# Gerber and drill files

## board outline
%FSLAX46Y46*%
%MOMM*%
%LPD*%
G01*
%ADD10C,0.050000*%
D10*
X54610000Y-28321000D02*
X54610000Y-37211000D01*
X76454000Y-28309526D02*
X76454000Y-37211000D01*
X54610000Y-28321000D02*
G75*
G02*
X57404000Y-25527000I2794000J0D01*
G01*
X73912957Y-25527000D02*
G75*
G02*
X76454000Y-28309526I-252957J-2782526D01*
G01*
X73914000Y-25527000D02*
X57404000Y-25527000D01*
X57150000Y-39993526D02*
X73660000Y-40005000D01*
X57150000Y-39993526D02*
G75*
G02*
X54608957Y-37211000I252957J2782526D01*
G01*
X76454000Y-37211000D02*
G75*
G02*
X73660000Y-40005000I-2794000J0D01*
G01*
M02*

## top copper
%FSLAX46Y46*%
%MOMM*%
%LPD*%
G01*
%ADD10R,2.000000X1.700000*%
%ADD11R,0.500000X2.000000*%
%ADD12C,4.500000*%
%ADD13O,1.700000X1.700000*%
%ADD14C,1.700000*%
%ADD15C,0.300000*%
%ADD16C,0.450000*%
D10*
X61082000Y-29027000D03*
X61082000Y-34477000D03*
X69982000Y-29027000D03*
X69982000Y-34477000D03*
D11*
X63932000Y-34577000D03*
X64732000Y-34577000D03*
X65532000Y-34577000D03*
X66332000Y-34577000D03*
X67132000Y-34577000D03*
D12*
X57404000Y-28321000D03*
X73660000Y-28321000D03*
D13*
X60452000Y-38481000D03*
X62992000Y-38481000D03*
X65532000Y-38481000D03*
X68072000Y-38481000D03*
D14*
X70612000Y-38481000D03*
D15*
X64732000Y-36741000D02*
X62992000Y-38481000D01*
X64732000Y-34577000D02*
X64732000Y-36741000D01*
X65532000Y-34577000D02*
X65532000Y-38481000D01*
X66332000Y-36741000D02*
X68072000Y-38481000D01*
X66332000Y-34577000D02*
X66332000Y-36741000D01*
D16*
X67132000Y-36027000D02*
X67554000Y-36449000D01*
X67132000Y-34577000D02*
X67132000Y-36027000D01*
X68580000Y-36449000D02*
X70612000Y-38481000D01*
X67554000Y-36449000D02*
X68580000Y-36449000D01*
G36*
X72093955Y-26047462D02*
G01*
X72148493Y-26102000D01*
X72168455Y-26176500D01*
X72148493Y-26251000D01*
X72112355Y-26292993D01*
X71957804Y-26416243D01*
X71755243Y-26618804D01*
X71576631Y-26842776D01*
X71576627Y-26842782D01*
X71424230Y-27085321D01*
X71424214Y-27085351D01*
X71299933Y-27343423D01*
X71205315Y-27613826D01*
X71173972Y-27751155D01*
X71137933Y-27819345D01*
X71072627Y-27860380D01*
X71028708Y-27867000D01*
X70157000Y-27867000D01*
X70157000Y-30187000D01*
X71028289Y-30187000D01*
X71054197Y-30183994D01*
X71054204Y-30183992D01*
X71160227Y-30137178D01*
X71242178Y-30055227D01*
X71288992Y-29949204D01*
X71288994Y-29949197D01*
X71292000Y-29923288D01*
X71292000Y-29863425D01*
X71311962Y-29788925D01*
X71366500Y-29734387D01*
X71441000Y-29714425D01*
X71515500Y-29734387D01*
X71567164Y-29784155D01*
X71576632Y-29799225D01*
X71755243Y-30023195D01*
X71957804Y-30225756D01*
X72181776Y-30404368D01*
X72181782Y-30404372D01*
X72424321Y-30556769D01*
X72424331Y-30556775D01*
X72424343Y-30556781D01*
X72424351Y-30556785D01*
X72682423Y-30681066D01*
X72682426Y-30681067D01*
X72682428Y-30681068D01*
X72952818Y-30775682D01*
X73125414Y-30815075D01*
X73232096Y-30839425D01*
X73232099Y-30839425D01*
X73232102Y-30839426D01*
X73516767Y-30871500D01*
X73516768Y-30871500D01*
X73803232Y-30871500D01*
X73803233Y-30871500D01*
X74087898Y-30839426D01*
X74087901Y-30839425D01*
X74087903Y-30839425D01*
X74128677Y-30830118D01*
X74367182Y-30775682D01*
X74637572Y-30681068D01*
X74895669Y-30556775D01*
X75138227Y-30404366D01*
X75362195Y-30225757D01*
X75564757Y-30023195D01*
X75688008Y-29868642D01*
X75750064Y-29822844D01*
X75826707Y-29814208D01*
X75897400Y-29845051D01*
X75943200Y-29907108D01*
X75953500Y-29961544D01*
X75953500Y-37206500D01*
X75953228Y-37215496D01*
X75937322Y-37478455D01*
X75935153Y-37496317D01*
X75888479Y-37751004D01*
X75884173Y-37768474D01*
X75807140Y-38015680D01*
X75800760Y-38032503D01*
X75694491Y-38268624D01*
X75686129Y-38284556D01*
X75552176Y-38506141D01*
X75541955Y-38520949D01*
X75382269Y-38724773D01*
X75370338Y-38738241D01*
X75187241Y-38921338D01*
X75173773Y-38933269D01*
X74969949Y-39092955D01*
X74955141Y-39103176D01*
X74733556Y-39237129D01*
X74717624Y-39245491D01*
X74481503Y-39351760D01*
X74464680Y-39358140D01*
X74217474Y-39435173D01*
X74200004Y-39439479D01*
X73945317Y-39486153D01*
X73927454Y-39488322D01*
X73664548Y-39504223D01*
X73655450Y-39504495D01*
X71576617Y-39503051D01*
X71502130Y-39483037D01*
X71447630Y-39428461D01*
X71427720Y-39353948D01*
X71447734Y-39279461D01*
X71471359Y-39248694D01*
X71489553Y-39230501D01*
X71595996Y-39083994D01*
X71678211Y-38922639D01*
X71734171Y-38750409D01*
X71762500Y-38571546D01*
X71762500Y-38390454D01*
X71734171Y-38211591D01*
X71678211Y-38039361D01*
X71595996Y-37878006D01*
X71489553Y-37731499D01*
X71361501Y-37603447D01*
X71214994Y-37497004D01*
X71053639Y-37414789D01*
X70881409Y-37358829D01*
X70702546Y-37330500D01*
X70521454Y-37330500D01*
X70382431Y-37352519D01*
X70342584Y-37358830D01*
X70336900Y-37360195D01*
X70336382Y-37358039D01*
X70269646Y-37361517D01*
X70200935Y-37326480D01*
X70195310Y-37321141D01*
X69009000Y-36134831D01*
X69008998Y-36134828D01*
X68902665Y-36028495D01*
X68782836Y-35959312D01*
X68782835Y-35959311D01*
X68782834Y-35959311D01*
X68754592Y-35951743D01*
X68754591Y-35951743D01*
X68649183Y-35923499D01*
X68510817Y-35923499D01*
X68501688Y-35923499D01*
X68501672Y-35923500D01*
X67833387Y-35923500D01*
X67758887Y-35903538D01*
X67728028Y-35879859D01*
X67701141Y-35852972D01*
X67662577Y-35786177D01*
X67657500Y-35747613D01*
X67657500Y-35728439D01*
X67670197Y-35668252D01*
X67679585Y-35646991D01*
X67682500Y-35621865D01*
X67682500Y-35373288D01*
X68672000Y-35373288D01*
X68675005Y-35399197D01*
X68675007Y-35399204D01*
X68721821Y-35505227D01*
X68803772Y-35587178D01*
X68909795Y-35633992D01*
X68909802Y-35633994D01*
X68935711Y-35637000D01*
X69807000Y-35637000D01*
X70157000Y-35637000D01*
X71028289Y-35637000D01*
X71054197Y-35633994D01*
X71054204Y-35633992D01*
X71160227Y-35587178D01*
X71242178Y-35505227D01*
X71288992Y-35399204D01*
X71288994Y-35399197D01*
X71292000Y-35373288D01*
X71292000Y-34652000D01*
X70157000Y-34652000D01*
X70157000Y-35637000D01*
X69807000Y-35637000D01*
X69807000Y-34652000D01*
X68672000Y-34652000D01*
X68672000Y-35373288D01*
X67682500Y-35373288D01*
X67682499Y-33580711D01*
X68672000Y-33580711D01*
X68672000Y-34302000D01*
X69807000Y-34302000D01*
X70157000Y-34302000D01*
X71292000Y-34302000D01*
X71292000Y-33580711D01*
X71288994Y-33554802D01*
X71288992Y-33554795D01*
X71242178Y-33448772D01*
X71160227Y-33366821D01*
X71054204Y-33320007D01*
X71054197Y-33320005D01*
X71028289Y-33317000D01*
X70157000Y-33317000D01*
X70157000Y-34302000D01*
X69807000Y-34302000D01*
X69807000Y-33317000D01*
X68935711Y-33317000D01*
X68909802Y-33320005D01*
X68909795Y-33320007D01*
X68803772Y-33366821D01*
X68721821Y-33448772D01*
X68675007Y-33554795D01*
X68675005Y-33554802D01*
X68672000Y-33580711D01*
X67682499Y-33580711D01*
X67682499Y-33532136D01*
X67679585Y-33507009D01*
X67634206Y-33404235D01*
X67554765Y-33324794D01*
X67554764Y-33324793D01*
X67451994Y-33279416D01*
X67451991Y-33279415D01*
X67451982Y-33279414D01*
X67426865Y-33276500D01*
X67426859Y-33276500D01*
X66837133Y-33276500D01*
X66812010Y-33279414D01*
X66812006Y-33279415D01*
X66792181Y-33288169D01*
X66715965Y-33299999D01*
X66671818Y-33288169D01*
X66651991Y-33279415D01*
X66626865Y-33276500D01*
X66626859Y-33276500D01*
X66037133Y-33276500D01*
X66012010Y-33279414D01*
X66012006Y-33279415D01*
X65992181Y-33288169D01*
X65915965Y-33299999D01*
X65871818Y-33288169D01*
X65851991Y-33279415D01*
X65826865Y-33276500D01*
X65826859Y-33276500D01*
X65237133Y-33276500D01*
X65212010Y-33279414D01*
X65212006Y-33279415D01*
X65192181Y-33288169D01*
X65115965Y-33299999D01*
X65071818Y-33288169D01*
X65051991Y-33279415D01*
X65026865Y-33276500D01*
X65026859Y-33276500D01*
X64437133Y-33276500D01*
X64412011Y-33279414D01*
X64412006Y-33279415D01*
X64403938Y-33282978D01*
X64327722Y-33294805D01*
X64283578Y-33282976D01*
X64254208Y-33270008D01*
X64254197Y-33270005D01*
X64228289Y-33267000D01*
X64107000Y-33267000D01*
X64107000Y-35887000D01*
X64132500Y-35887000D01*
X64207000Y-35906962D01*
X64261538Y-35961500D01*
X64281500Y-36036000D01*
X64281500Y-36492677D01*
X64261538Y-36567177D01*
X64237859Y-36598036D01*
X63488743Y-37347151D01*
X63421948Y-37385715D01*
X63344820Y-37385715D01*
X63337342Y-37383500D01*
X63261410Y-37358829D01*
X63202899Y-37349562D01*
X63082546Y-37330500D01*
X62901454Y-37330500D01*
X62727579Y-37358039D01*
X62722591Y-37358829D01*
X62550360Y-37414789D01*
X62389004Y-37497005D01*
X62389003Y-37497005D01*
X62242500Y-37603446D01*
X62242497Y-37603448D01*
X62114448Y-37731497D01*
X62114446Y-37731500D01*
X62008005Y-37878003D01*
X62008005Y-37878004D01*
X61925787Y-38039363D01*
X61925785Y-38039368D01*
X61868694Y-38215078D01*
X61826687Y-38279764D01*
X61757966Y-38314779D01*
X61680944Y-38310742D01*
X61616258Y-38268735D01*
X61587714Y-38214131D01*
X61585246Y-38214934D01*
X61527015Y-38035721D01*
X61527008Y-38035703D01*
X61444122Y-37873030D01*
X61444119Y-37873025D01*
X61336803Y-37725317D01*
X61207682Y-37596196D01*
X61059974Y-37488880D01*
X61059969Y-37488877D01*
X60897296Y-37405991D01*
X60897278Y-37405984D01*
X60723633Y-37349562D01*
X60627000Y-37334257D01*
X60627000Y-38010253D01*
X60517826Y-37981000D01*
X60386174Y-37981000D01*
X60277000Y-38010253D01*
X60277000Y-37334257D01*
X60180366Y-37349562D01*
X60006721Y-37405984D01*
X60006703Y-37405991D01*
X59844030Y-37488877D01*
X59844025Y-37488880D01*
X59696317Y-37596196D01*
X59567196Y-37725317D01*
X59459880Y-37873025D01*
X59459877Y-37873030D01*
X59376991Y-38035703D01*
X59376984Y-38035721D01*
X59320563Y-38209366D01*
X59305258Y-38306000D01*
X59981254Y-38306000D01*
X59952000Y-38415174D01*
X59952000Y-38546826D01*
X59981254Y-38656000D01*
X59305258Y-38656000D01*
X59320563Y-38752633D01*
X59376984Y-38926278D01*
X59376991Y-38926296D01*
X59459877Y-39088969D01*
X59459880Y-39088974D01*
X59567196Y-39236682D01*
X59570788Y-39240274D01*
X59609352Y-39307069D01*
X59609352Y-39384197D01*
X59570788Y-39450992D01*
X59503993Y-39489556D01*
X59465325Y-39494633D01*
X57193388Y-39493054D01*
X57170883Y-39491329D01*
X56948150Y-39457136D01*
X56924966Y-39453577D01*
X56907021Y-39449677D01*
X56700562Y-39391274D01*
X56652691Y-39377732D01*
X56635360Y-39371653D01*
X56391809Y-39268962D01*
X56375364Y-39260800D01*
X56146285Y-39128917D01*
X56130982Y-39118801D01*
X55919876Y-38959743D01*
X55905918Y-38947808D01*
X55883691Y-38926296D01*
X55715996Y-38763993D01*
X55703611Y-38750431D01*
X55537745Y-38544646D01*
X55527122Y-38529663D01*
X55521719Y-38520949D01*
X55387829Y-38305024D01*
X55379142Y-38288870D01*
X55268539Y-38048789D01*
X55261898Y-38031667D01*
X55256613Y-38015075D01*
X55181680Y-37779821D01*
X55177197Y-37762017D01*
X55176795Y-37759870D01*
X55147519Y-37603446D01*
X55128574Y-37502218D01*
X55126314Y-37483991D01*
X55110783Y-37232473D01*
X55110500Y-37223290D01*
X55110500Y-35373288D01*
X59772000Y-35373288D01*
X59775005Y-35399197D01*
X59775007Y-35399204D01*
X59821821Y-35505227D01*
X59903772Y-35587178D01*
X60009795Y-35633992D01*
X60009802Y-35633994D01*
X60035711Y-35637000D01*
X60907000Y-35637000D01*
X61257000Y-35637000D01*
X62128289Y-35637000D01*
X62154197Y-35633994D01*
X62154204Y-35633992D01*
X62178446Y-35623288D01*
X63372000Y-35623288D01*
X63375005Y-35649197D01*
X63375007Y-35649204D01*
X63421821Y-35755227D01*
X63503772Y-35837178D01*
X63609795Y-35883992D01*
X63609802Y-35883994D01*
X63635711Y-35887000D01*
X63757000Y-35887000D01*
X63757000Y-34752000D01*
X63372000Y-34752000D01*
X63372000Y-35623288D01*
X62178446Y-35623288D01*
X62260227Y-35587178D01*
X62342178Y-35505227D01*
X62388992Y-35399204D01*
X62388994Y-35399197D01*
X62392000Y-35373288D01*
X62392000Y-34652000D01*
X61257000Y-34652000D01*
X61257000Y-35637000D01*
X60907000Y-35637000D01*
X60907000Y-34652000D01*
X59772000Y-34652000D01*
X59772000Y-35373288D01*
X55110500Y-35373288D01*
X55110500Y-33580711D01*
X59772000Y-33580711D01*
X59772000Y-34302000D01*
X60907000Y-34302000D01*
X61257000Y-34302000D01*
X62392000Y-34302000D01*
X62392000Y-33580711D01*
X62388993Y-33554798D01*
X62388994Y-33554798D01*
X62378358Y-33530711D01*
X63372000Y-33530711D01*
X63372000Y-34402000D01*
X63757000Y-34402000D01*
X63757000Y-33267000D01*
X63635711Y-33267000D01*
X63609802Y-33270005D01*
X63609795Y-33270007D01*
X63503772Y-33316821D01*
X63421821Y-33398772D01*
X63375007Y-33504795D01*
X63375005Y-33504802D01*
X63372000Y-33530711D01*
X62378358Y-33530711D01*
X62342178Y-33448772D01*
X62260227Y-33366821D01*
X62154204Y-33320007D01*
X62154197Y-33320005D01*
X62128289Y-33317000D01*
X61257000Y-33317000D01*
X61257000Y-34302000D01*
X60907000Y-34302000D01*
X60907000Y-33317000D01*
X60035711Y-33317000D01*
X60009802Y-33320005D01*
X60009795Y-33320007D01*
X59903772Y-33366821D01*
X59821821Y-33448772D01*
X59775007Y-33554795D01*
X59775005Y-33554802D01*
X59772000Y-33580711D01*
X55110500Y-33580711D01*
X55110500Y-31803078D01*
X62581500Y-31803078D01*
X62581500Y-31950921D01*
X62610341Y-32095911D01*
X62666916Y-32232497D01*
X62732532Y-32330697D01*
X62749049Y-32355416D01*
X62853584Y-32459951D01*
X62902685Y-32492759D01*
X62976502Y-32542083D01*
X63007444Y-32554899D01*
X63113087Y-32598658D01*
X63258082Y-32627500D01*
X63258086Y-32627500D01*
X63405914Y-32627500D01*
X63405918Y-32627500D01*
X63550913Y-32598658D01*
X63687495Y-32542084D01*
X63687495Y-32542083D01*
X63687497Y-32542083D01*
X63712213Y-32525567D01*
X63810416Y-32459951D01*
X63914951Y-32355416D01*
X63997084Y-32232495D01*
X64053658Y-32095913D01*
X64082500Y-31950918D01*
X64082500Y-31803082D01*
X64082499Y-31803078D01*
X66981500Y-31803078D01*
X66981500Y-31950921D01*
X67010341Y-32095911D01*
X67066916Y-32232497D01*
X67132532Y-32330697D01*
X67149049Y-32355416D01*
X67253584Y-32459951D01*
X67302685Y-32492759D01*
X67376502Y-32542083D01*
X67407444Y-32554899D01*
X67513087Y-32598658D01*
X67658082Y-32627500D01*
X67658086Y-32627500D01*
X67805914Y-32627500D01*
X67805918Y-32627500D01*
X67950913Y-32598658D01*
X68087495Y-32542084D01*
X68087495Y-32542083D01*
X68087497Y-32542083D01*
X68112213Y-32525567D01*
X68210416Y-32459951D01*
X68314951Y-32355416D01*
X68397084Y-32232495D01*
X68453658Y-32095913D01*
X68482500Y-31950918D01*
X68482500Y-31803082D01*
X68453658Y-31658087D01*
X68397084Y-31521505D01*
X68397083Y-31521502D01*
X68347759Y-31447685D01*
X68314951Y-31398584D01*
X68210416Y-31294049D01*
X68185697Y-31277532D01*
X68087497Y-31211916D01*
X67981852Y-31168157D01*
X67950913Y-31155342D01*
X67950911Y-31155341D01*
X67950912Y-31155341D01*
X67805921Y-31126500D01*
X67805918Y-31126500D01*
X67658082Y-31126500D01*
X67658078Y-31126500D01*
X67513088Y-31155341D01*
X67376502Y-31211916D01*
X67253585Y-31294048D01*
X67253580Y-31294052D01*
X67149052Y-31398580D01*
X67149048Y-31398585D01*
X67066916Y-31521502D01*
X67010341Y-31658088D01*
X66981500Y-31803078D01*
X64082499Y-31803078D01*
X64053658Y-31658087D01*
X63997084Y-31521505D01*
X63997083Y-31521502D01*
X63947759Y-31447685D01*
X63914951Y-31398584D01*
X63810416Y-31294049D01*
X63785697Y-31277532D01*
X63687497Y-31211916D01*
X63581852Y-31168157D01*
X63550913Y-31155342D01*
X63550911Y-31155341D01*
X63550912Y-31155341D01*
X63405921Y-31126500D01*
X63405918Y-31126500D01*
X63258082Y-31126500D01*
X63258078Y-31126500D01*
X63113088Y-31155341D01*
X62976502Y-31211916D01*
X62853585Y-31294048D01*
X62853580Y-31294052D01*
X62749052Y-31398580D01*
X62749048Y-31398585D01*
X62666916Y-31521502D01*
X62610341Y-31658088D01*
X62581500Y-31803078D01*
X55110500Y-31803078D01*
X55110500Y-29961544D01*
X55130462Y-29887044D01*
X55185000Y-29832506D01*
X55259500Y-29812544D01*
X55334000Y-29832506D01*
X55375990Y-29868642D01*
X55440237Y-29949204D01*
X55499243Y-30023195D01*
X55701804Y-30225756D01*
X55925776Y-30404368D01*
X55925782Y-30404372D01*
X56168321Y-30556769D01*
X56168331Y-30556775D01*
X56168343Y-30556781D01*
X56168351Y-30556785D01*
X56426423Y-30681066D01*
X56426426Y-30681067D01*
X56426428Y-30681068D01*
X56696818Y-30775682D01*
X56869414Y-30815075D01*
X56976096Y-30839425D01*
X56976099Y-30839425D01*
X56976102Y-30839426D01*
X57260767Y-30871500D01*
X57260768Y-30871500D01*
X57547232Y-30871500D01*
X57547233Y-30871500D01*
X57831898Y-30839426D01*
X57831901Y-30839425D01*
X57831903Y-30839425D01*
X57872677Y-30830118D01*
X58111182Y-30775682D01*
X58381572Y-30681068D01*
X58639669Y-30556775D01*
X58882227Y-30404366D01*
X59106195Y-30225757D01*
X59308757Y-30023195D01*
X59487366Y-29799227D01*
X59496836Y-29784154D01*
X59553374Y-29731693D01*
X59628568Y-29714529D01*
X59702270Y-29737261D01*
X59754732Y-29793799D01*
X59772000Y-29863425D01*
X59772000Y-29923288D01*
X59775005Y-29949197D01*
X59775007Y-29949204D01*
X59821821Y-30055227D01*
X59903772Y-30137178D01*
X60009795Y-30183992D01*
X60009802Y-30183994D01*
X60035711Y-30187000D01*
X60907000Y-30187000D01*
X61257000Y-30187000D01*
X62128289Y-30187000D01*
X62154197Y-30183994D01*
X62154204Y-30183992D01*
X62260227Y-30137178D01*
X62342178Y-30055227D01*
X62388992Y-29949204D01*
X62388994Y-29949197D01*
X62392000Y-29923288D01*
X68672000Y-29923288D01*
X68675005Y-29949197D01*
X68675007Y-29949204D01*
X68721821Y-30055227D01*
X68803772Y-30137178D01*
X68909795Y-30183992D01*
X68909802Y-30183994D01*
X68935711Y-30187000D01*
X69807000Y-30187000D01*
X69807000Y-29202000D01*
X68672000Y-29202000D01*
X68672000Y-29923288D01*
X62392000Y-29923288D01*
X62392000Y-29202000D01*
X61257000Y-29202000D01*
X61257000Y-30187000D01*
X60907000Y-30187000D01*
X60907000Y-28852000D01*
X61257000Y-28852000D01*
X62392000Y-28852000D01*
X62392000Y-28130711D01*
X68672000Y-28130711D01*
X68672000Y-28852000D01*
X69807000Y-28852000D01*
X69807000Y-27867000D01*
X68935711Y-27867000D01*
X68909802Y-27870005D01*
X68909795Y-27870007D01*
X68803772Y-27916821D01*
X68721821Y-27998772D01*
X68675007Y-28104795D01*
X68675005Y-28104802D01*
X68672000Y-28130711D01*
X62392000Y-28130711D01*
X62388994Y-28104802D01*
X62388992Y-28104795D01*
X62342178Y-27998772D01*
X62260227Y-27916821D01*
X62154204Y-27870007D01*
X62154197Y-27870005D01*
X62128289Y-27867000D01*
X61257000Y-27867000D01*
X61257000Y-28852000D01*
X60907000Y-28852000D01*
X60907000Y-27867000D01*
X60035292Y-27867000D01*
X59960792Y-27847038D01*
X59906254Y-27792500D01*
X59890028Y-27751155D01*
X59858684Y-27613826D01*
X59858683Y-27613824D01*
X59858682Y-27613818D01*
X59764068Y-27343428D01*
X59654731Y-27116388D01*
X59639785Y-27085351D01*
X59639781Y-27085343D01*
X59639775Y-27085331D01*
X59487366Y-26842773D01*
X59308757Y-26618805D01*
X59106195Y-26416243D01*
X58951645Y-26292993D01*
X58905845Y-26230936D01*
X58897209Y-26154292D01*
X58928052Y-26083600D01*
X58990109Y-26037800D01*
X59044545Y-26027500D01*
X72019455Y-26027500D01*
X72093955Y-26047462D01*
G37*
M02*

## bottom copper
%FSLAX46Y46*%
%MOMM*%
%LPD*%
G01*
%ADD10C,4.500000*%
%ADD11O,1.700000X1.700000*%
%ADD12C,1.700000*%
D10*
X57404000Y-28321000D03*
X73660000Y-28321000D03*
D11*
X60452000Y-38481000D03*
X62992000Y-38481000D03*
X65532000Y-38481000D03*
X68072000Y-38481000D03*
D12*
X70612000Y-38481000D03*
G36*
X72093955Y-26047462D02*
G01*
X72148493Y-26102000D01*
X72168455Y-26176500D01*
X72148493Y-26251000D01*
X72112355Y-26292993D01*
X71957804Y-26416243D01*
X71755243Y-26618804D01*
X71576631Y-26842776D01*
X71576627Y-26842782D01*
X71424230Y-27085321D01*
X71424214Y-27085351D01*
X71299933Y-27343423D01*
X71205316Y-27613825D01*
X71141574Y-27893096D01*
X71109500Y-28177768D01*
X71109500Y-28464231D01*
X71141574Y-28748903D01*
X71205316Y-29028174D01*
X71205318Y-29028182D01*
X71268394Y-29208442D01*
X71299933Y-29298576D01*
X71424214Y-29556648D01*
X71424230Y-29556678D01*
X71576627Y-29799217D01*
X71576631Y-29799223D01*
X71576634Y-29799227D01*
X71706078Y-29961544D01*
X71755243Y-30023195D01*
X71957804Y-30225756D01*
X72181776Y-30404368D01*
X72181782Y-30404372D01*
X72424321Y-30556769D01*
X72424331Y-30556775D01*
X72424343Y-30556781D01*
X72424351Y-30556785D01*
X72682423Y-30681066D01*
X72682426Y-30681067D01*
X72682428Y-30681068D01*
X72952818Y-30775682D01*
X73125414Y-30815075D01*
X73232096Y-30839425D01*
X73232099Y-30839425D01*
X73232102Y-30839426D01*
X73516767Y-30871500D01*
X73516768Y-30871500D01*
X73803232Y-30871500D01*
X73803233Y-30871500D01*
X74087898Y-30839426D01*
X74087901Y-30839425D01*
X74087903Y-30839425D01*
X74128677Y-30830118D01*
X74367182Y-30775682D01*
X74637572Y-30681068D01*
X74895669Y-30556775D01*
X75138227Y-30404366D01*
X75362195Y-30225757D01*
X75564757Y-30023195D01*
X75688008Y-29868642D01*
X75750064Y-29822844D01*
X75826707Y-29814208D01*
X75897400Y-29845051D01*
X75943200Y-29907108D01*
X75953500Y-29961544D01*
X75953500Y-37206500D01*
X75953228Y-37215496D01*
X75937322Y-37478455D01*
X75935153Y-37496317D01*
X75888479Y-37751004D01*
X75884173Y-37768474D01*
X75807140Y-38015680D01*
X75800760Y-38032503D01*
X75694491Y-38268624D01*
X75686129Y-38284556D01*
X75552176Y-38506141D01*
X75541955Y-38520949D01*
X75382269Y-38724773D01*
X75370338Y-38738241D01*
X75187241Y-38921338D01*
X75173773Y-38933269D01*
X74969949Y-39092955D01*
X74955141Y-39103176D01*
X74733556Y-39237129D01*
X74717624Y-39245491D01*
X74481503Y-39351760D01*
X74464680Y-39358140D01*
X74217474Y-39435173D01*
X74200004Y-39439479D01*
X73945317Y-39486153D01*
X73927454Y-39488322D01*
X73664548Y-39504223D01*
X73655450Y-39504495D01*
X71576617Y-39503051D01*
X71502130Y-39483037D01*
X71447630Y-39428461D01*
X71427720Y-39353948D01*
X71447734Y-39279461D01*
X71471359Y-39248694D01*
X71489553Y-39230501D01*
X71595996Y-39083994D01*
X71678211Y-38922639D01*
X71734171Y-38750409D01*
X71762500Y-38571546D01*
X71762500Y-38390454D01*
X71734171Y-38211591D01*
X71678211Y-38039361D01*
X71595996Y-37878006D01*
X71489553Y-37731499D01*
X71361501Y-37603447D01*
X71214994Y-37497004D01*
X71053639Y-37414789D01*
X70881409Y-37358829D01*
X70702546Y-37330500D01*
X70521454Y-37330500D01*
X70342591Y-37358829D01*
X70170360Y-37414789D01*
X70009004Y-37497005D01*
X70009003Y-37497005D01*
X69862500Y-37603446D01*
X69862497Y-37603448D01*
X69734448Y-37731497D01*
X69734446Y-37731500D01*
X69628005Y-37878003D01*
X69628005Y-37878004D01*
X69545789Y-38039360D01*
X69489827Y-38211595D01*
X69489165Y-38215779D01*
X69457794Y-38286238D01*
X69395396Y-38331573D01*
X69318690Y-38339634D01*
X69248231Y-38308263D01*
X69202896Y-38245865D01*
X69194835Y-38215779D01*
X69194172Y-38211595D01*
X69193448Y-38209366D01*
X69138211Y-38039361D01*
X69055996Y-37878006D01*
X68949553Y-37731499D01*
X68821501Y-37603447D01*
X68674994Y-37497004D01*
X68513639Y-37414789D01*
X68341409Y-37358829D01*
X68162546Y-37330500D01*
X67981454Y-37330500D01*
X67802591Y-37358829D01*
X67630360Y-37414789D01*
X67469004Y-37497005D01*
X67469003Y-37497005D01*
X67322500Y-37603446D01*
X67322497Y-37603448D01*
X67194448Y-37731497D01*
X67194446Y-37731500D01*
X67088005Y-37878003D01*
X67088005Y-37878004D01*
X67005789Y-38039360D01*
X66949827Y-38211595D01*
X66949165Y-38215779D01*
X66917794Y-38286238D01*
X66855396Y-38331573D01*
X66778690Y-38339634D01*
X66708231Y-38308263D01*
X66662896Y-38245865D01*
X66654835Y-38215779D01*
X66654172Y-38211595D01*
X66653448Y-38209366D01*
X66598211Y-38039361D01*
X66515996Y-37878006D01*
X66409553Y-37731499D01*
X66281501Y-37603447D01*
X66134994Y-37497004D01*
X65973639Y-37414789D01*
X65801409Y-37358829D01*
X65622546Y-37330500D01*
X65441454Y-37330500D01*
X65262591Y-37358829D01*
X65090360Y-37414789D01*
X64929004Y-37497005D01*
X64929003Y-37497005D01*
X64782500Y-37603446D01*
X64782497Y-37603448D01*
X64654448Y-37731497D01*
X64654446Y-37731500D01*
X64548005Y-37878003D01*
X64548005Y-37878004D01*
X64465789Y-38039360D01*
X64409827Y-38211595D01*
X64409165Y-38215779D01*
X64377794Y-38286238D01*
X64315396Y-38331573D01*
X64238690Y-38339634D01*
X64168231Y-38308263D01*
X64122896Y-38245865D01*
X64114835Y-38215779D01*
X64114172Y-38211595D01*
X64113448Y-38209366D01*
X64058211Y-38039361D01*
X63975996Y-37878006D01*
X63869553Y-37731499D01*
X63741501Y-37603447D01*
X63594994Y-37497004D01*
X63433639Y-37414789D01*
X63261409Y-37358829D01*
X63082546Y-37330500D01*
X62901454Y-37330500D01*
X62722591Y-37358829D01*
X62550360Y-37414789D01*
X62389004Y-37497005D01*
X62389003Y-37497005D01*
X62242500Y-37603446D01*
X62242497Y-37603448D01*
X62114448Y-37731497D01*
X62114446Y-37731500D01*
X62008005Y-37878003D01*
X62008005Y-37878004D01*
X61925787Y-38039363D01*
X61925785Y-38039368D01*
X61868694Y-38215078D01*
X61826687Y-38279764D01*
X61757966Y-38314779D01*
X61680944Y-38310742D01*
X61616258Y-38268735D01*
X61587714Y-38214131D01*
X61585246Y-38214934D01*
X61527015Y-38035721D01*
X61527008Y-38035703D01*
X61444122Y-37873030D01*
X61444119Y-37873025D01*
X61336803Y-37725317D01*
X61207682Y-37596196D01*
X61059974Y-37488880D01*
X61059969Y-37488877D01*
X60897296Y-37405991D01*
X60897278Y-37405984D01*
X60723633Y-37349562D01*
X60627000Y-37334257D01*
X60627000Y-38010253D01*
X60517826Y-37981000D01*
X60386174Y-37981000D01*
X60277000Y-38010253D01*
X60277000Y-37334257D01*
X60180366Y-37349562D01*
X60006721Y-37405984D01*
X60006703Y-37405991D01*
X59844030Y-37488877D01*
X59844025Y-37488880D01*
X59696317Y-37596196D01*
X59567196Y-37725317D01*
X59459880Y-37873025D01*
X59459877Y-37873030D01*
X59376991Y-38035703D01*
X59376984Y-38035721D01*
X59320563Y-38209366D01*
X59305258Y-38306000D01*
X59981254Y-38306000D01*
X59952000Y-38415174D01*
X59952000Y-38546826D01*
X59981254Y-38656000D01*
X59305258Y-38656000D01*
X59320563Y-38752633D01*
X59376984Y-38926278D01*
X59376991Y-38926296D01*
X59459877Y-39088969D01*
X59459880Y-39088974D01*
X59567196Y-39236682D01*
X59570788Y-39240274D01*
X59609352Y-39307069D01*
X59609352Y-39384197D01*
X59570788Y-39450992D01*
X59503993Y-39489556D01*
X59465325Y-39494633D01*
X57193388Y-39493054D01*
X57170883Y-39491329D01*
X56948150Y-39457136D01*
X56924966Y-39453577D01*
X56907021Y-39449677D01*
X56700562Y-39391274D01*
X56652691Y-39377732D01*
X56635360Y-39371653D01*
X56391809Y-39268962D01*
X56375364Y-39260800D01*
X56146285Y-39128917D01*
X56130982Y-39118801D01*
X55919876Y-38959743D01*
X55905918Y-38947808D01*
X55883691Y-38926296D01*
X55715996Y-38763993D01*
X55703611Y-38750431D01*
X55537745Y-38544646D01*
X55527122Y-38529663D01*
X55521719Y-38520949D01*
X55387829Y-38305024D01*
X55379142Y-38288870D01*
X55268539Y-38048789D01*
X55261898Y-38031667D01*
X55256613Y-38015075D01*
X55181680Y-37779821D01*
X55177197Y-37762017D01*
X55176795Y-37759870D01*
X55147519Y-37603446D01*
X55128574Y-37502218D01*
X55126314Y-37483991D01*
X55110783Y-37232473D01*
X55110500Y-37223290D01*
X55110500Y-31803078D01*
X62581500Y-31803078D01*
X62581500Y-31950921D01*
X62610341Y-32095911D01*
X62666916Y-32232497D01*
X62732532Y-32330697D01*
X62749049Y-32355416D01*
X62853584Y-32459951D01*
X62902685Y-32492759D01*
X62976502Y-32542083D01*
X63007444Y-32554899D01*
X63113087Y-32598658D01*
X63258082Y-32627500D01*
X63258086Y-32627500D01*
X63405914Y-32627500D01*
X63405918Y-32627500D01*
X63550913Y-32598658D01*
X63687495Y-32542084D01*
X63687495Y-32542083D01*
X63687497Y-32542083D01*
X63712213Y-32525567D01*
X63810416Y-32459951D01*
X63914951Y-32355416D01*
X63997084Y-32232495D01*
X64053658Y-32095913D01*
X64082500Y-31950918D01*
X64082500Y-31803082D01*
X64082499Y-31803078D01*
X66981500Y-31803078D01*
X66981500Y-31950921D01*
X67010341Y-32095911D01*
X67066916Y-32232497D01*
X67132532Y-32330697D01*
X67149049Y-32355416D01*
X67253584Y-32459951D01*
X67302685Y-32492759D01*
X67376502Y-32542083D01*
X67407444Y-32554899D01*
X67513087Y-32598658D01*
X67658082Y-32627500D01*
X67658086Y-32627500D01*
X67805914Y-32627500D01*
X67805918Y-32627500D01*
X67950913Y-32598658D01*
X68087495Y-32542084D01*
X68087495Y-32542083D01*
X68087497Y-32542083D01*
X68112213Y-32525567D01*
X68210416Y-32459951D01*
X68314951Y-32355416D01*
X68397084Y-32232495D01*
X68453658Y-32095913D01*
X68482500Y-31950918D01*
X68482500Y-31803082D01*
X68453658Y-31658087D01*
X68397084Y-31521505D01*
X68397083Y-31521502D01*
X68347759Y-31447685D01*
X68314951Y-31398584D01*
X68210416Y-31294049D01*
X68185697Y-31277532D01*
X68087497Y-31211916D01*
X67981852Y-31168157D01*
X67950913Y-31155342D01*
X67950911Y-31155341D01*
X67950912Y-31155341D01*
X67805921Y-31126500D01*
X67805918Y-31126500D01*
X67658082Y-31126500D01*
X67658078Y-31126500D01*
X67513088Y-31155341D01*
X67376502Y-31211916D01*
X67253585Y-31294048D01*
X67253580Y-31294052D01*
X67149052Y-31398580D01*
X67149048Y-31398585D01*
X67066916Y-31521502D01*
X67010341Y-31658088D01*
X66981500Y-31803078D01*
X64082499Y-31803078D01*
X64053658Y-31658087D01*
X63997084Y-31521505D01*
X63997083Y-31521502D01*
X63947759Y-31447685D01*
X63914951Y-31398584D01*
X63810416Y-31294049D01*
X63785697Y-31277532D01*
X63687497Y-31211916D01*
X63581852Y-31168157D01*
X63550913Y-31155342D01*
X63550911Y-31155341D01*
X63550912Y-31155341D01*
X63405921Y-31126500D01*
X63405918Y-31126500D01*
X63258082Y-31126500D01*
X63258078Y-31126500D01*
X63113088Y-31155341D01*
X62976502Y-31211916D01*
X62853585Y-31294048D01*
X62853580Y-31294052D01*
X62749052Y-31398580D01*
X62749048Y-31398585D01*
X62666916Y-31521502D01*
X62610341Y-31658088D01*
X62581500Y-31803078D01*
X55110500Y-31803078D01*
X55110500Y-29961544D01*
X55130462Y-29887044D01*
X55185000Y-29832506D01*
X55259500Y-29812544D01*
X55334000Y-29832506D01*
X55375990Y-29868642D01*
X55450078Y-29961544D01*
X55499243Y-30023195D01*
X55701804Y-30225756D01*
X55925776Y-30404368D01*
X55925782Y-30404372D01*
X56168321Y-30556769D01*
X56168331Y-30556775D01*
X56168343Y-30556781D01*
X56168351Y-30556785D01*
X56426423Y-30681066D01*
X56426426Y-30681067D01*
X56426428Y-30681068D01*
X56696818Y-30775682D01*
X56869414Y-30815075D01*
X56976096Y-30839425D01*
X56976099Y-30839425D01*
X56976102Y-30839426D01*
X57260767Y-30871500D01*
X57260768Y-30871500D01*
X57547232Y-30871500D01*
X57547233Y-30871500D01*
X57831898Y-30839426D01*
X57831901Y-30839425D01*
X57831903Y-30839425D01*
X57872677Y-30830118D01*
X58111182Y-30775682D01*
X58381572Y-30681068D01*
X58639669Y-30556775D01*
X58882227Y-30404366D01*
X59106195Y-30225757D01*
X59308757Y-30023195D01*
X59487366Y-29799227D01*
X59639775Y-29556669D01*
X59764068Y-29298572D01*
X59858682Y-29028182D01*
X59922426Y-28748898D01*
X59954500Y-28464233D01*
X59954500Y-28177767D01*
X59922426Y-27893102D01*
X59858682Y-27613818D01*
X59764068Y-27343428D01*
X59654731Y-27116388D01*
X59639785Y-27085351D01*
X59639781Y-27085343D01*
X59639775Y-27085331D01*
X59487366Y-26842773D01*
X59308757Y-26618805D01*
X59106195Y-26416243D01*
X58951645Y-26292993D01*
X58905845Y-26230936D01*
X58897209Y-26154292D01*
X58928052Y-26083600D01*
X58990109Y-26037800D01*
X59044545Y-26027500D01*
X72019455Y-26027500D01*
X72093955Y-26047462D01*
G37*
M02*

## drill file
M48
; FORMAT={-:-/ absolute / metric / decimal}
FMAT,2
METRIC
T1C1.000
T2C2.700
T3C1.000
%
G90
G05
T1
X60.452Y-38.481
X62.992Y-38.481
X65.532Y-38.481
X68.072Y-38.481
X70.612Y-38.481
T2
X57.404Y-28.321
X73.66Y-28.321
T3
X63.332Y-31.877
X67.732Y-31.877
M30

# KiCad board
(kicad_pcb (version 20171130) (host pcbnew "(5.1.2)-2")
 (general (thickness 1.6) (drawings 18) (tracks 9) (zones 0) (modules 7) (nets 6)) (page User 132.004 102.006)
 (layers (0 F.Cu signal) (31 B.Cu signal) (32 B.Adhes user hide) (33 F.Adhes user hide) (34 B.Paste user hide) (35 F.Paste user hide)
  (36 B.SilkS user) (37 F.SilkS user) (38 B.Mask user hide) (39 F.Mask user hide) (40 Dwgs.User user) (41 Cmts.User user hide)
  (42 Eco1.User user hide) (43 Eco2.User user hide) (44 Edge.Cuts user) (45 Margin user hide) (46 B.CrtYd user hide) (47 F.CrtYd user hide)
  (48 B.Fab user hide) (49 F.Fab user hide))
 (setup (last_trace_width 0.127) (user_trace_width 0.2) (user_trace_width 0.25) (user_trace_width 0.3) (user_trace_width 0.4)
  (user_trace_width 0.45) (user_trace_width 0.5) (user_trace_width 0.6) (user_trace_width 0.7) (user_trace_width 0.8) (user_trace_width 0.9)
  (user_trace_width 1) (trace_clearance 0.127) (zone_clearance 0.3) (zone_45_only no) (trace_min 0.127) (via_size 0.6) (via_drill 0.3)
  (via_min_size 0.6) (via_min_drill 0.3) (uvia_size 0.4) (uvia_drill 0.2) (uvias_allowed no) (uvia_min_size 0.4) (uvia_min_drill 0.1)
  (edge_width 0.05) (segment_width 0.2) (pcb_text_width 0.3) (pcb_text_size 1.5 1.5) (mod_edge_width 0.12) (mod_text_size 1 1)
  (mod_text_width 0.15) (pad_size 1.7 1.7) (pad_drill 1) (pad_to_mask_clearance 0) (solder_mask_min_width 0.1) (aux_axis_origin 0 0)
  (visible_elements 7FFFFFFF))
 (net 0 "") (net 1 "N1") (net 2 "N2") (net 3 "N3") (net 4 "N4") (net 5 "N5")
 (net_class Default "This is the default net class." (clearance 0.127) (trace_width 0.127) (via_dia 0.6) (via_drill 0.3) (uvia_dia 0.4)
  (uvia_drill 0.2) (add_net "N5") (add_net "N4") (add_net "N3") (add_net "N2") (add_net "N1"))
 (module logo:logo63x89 (layer B.Cu) (at 65.532 29.083 180)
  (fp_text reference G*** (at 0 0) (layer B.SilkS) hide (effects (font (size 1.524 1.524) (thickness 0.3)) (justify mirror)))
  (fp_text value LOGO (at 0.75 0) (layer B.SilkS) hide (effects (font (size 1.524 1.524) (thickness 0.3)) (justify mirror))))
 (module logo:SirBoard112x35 (layer B.Cu) (at 65.532 34.671 180)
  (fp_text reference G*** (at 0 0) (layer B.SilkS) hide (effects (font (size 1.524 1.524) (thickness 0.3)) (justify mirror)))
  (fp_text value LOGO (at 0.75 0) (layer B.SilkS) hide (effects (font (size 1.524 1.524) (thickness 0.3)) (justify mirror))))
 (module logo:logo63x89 (layer F.Cu) (at 57.404 34.925)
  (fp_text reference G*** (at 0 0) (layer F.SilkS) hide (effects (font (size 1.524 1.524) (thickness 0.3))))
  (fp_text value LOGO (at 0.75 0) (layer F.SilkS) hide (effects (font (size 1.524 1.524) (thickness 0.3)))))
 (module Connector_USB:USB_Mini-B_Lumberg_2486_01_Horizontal (layer F.Cu) (at 65.532 31.877 180)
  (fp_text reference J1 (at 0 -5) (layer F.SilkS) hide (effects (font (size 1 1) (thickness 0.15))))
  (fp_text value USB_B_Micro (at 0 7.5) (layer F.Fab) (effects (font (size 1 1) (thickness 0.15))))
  (pad "" np_thru_hole circle (at 2.2 0 180) (size 1 1) (drill 1) (layers *.Cu *.Mask))
  (pad "" np_thru_hole circle (at -2.2 0 180) (size 1 1) (drill 1) (layers *.Cu *.Mask))
  (pad 6 smd rect (at 4.45 2.85 180) (size 2 1.7) (layers F.Cu F.Paste F.Mask) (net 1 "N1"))
  (pad 6 smd rect (at 4.45 -2.6 180) (size 2 1.7) (layers F.Cu F.Paste F.Mask) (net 1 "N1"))
  (pad 6 smd rect (at -4.45 2.85 180) (size 2 1.7) (layers F.Cu F.Paste F.Mask) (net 1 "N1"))
  (pad 6 smd rect (at -4.45 -2.6 180) (size 2 1.7) (layers F.Cu F.Paste F.Mask) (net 1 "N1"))
  (pad 5 smd rect (at 1.6 -2.7 180) (size 0.5 2) (layers F.Cu F.Paste F.Mask) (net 1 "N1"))
  (pad 4 smd rect (at 0.8 -2.7 180) (size 0.5 2) (layers F.Cu F.Paste F.Mask) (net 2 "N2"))
  (pad 3 smd rect (at 0 -2.7 180) (size 0.5 2) (layers F.Cu F.Paste F.Mask) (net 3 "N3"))
  (pad 2 smd rect (at -0.8 -2.7 180) (size 0.5 2) (layers F.Cu F.Paste F.Mask) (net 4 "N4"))
  (pad 1 smd rect (at -1.6 -2.7 180) (size 0.5 2) (layers F.Cu F.Paste F.Mask) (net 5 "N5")))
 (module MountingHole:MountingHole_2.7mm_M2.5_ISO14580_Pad (layer F.Cu) (at 57.404 28.321 270)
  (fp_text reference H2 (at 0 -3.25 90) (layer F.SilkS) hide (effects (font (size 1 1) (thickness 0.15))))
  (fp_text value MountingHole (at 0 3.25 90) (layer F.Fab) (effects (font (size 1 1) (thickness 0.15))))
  (pad 1 thru_hole circle (at 0 0 270) (size 4.5 4.5) (drill 2.7) (layers *.Cu *.Mask)))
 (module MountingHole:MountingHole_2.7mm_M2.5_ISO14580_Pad (layer F.Cu) (at 73.66 28.321 270)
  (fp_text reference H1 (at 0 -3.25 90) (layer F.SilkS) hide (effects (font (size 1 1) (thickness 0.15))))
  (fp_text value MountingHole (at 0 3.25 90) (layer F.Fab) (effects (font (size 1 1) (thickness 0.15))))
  (pad 1 thru_hole circle (at 0 0 270) (size 4.5 4.5) (drill 2.7) (layers *.Cu *.Mask)))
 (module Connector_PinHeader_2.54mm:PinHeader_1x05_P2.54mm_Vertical (layer B.Cu) (at 70.612 38.481 90)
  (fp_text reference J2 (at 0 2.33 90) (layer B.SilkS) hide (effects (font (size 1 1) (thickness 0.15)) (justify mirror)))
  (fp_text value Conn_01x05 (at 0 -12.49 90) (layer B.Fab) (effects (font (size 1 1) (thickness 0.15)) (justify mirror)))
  (pad 5 thru_hole oval (at 0 -10.16 90) (size 1.7 1.7) (drill 1) (layers *.Cu *.Mask) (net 1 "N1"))
  (pad 4 thru_hole oval (at 0 -7.62 90) (size 1.7 1.7) (drill 1) (layers *.Cu *.Mask) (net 2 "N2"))
  (pad 3 thru_hole oval (at 0 -5.08 90) (size 1.7 1.7) (drill 1) (layers *.Cu *.Mask) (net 3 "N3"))
  (pad 2 thru_hole oval (at 0 -2.54 90) (size 1.7 1.7) (drill 1) (layers *.Cu *.Mask) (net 4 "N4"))
  (pad 1 thru_hole circle (at 0 0 90) (size 1.7 1.7) (drill 1) (layers *.Cu *.Mask) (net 5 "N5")))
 (gr_line (start 54.61 28.321) (end 54.61 37.211) (layer Edge.Cuts) (width 0.05))
 (gr_line (start 76.454 28.309526) (end 76.454 37.211) (layer Edge.Cuts) (width 0.05))
 (gr_arc (start 57.404 28.321) (end 57.404 25.527) (angle -90) (layer Edge.Cuts) (width 0.05))
 (gr_arc (start 73.66 28.309526) (end 76.454 28.309526) (angle -84.80557109) (layer Edge.Cuts) (width 0.05))
 (gr_line (start 73.914 25.527) (end 57.404 25.527) (layer Edge.Cuts) (width 0.05))
 (gr_line (start 57.15 39.993526) (end 73.66 40.005) (layer Edge.Cuts) (width 0.05))
 (gr_arc (start 57.402957 37.211) (end 54.608957 37.211) (angle -84.80557109) (layer Edge.Cuts) (width 0.05))
 (gr_arc (start 73.66 37.211) (end 73.66 40.005) (angle -90) (layer Edge.Cuts) (width 0.05))
 (segment (start 64.732 36.741) (end 62.992 38.481) (width 0.3) (layer F.Cu) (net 2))
 (segment (start 64.732 34.577) (end 64.732 36.741) (width 0.3) (layer F.Cu) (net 2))
 (segment (start 65.532 34.577) (end 65.532 38.481) (width 0.3) (layer F.Cu) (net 3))
 (segment (start 66.332 36.741) (end 68.072 38.481) (width 0.3) (layer F.Cu) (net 4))
 (segment (start 66.332 34.577) (end 66.332 36.741) (width 0.3) (layer F.Cu) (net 4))
 (segment (start 67.132 36.027) (end 67.554 36.449) (width 0.45) (layer F.Cu) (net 5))
 (segment (start 67.132 34.577) (end 67.132 36.027) (width 0.45) (layer F.Cu) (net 5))
 (segment (start 68.58 36.449) (end 70.612 38.481) (width 0.45) (layer F.Cu) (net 5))
 (segment (start 67.554 36.449) (end 68.58 36.449) (width 0.45) (layer F.Cu) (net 5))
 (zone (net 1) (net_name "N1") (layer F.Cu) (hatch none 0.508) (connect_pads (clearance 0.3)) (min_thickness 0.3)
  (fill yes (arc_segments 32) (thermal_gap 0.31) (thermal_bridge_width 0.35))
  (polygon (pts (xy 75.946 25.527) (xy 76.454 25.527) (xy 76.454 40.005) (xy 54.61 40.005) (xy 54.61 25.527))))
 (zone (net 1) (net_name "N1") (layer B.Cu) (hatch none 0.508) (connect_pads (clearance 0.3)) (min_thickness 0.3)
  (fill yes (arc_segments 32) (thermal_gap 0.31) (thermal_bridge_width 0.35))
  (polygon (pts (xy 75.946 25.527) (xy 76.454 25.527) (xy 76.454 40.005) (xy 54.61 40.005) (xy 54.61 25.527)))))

